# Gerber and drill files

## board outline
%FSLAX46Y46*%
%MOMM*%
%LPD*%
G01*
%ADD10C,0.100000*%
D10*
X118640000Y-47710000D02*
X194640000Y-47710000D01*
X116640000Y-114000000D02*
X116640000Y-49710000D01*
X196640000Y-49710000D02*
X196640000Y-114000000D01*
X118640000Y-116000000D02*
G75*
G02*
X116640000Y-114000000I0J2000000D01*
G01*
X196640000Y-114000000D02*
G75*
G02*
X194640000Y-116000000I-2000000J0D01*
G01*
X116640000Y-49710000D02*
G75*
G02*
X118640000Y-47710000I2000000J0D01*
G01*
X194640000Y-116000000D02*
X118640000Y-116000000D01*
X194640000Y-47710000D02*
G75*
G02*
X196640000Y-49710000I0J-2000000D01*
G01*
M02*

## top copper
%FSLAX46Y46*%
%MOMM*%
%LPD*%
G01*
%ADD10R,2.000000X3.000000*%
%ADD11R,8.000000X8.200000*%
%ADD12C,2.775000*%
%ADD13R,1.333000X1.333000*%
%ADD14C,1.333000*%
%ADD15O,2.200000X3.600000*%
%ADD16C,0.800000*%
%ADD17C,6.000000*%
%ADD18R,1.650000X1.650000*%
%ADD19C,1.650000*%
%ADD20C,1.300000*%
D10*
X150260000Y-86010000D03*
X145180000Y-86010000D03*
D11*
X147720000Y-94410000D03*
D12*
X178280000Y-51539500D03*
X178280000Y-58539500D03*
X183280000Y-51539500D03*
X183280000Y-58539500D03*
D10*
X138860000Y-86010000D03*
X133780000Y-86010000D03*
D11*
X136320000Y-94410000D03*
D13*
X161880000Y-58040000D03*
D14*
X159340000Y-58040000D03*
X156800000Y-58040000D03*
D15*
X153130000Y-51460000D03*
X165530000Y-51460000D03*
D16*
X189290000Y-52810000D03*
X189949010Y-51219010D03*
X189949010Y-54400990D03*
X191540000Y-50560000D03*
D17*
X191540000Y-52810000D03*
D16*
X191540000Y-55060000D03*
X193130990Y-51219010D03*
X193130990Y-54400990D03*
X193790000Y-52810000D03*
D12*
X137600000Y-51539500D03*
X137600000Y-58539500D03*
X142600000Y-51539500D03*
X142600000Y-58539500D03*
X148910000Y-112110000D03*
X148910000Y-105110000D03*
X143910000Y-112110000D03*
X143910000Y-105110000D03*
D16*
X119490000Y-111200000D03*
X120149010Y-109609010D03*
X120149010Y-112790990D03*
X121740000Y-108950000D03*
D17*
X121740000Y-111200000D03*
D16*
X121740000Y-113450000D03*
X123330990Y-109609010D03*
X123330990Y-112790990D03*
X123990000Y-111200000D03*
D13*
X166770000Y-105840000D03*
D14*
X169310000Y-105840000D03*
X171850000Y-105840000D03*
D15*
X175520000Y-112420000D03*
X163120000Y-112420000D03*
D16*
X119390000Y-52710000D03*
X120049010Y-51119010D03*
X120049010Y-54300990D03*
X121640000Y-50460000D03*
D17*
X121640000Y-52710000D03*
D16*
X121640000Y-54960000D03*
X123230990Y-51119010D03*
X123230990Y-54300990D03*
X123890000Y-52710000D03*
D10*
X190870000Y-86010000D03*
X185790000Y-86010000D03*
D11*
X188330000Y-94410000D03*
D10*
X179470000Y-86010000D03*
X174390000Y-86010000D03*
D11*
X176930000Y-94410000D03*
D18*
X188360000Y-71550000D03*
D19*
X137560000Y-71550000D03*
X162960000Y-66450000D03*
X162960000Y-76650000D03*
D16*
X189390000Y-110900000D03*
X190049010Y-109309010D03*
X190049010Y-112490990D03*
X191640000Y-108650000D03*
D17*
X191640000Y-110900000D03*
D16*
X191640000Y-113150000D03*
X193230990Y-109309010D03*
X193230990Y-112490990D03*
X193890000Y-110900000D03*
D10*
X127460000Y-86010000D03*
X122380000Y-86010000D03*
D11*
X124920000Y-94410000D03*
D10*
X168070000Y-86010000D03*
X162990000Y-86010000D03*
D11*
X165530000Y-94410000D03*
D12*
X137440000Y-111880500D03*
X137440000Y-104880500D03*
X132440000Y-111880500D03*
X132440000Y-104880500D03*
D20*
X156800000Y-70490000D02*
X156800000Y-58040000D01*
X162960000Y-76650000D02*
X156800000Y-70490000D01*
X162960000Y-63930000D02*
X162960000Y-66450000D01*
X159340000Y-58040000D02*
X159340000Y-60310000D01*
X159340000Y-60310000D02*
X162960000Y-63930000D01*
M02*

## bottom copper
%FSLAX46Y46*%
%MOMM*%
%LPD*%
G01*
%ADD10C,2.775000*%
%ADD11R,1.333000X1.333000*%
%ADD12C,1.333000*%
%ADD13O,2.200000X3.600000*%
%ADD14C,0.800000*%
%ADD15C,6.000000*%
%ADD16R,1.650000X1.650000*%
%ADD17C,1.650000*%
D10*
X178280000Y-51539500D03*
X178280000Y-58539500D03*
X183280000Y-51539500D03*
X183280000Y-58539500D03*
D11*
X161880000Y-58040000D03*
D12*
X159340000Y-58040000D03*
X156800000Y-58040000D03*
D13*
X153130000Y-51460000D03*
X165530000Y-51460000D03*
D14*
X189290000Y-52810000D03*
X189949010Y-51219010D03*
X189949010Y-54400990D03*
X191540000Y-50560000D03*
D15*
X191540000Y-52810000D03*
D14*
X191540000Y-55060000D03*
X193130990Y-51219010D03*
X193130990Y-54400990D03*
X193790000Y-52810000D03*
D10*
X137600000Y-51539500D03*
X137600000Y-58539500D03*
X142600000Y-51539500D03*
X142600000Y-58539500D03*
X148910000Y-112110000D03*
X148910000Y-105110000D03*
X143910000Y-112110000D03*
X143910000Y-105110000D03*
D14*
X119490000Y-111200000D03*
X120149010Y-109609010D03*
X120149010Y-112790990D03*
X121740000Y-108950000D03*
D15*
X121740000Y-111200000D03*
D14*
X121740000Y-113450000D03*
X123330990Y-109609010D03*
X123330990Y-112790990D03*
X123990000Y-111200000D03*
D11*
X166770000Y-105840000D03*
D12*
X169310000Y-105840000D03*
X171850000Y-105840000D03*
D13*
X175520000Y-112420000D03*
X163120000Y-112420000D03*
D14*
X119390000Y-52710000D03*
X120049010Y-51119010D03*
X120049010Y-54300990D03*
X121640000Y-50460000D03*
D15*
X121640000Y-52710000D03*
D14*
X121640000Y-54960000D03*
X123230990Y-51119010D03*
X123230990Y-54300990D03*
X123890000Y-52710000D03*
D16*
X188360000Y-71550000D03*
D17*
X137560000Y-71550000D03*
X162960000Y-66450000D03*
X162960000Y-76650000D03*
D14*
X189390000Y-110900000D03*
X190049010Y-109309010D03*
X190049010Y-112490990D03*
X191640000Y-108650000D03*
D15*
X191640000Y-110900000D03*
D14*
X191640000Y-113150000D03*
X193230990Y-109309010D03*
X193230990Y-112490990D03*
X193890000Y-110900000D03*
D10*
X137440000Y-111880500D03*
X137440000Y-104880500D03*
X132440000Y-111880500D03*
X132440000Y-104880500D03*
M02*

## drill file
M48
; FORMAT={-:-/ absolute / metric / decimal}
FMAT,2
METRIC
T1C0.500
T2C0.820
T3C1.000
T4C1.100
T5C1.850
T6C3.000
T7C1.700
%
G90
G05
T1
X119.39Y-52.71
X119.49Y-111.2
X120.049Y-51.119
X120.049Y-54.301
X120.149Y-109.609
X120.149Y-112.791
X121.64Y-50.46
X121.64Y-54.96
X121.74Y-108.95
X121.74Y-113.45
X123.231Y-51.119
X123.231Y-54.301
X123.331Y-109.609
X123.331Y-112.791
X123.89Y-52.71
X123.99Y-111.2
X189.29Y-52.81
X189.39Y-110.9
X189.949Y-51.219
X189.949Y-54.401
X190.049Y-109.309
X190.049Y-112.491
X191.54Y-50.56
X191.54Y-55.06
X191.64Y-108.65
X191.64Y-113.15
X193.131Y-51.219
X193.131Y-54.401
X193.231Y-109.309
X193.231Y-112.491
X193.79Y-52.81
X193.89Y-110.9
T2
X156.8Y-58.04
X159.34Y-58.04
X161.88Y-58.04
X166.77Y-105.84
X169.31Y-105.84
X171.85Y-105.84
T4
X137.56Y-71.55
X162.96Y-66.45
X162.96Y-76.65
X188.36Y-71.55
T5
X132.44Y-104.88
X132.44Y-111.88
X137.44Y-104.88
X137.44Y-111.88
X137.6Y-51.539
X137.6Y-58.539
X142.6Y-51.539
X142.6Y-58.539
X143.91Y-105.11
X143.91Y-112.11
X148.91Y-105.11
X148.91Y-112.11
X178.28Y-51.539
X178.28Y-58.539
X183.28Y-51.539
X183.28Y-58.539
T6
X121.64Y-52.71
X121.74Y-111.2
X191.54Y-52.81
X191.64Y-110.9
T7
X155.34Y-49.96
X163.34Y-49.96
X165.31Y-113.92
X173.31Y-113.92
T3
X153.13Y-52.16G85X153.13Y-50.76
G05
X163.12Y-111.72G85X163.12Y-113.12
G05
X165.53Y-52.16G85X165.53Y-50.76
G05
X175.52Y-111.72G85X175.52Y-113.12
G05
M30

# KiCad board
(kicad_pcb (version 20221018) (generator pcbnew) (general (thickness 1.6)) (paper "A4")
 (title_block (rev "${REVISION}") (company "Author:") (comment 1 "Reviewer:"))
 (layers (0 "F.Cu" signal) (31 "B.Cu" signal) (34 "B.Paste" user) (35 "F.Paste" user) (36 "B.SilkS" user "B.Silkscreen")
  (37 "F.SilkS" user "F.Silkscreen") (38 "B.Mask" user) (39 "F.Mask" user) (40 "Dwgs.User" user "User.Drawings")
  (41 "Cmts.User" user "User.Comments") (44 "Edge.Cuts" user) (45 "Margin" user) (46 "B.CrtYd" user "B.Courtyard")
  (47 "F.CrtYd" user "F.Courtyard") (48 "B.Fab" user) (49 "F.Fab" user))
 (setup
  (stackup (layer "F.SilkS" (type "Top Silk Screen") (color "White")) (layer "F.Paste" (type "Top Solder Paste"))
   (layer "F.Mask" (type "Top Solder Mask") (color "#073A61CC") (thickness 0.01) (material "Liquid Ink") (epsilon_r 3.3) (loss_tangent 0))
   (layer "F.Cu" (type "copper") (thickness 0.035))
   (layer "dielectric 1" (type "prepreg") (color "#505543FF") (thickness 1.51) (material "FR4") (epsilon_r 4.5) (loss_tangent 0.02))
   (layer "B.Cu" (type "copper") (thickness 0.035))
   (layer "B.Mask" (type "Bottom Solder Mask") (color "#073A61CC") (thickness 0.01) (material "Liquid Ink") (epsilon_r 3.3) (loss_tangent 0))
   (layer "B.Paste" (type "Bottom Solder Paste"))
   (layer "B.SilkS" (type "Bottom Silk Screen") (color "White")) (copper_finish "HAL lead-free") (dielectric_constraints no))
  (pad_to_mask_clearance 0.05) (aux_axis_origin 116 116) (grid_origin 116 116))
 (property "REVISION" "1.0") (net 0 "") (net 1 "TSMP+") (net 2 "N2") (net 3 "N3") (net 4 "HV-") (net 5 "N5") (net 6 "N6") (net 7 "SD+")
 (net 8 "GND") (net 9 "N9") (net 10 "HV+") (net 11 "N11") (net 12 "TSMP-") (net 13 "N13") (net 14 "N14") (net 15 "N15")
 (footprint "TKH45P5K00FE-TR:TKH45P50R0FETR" (layer "F.Cu") (at 147.72 90.21 180)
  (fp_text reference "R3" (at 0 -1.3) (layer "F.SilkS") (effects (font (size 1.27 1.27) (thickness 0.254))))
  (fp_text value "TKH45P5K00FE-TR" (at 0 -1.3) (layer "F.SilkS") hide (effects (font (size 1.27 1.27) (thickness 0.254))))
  (pad "1" smd rect (at -2.54 4.2 180) (size 2 3) (layers "F.Cu" "F.Paste" "F.Mask") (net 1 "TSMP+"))
  (pad "2" smd rect (at 2.54 4.2 180) (size 2 3) (layers "F.Cu" "F.Paste" "F.Mask") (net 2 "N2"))
  (pad "3" smd rect (at 0 -4.2 180) (size 8 8.2) (layers "F.Cu" "F.Paste" "F.Mask") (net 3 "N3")))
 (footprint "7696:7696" (layer "F.Cu") (at 178.28 58.5395)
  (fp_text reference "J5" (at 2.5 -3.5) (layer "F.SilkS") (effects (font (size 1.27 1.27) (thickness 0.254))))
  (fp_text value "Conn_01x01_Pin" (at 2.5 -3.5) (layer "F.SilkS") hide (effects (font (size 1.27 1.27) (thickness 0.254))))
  (pad "1" thru_hole circle (at 0 -7) (size 2.775 2.775) (drill 1.85) (layers "*.Cu" "*.Mask") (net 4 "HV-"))
  (pad "1" thru_hole circle (at 0 0) (size 2.775 2.775) (drill 1.85) (layers "*.Cu" "*.Mask") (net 4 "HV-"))
  (pad "1" thru_hole circle (at 5 -7) (size 2.775 2.775) (drill 1.85) (layers "*.Cu" "*.Mask") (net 4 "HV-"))
  (pad "1" thru_hole circle (at 5 0) (size 2.775 2.775) (drill 1.85) (layers "*.Cu" "*.Mask") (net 4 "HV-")))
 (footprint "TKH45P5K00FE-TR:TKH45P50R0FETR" (layer "F.Cu") (at 136.32 90.21 180)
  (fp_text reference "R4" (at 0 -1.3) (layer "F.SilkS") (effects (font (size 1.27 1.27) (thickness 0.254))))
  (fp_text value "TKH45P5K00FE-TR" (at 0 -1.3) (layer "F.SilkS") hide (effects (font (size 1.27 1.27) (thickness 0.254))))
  (pad "1" smd rect (at -2.54 4.2 180) (size 2 3) (layers "F.Cu" "F.Paste" "F.Mask") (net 2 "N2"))
  (pad "2" smd rect (at 2.54 4.2 180) (size 2 3) (layers "F.Cu" "F.Paste" "F.Mask") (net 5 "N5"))
  (pad "3" smd rect (at 0 -4.2 180) (size 8 8.2) (layers "F.Cu" "F.Paste" "F.Mask") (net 3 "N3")))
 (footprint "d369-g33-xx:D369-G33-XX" (layer "F.Cu") (at 161.88 58.04 90)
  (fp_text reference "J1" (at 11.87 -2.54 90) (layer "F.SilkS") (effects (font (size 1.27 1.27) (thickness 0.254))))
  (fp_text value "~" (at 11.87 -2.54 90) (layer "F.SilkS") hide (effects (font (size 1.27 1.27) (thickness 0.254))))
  (pad "" np_thru_hole circle (at 8.08 -6.54 90) (size 1.7 1.7) (drill 1.7) (layers "*.Cu" "*.Mask"))
  (pad "" np_thru_hole circle (at 8.08 1.46 90) (size 1.7 1.7) (drill 1.7) (layers "*.Cu" "*.Mask"))
  (pad "1" thru_hole rect (at 0 0 90) (size 1.333 1.333) (drill 0.82) (layers "*.Cu" "*.Mask") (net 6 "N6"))
  (pad "2" thru_hole circle (at 0 -2.54 90) (size 1.333 1.333) (drill 0.82) (layers "*.Cu" "*.Mask") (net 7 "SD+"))
  (pad "3" thru_hole circle (at 0 -5.08 90) (size 1.333 1.333) (drill 0.82) (layers "*.Cu" "*.Mask") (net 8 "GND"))
  (pad "MH" thru_hole oval (at 6.58 -8.75 90) (size 3.6 2.2) (drill oval 2.4 1) (layers "*.Cu" "*.Mask"))
  (pad "MH" thru_hole oval (at 6.58 3.65 90) (size 3.6 2.2) (drill oval 2.4 1) (layers "*.Cu" "*.Mask")))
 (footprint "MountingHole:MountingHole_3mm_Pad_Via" (layer "F.Cu") (at 191.54 52.81)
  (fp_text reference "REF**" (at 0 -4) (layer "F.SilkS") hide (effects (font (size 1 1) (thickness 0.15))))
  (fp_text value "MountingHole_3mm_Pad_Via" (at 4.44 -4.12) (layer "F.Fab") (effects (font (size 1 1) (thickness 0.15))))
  (pad "1" thru_hole circle (at -2.25 0) (size 0.8 0.8) (drill 0.5) (layers "*.Cu" "*.Mask") (zone_connect 2))
  (pad "1" thru_hole circle (at -1.59099 -1.59099) (size 0.8 0.8) (drill 0.5) (layers "*.Cu" "*.Mask") (zone_connect 2))
  (pad "1" thru_hole circle (at -1.59099 1.59099) (size 0.8 0.8) (drill 0.5) (layers "*.Cu" "*.Mask") (zone_connect 2))
  (pad "1" thru_hole circle (at 0 -2.25) (size 0.8 0.8) (drill 0.5) (layers "*.Cu" "*.Mask") (zone_connect 2))
  (pad "1" thru_hole circle (at 0 0) (size 6 6) (drill 3) (layers "*.Cu" "*.Mask"))
  (pad "1" thru_hole circle (at 0 2.25) (size 0.8 0.8) (drill 0.5) (layers "*.Cu" "*.Mask") (zone_connect 2))
  (pad "1" thru_hole circle (at 1.59099 -1.59099) (size 0.8 0.8) (drill 0.5) (layers "*.Cu" "*.Mask") (zone_connect 2))
  (pad "1" thru_hole circle (at 1.59099 1.59099) (size 0.8 0.8) (drill 0.5) (layers "*.Cu" "*.Mask") (zone_connect 2))
  (pad "1" thru_hole circle (at 2.25 0) (size 0.8 0.8) (drill 0.5) (layers "*.Cu" "*.Mask") (zone_connect 2)))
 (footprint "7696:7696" (layer "F.Cu") (at 137.6 58.5395)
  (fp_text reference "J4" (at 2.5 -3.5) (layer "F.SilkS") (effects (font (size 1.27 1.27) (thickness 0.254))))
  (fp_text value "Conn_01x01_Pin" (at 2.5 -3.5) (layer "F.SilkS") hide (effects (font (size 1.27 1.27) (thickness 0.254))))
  (pad "1" thru_hole circle (at 0 -7) (size 2.775 2.775) (drill 1.85) (layers "*.Cu" "*.Mask") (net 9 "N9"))
  (pad "1" thru_hole circle (at 0 0) (size 2.775 2.775) (drill 1.85) (layers "*.Cu" "*.Mask") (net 9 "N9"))
  (pad "1" thru_hole circle (at 5 -7) (size 2.775 2.775) (drill 1.85) (layers "*.Cu" "*.Mask") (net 9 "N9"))
  (pad "1" thru_hole circle (at 5 0) (size 2.775 2.775) (drill 1.85) (layers "*.Cu" "*.Mask") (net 9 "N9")))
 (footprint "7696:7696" (layer "F.Cu") (at 148.91 105.11 180)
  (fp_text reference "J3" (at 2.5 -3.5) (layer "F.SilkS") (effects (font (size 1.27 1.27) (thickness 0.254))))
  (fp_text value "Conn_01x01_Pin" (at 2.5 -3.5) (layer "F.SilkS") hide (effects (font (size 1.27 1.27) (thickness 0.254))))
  (pad "1" thru_hole circle (at 0 -7 180) (size 2.775 2.775) (drill 1.85) (layers "*.Cu" "*.Mask") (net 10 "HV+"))
  (pad "1" thru_hole circle (at 0 0 180) (size 2.775 2.775) (drill 1.85) (layers "*.Cu" "*.Mask") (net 10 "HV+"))
  (pad "1" thru_hole circle (at 5 -7 180) (size 2.775 2.775) (drill 1.85) (layers "*.Cu" "*.Mask") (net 10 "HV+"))
  (pad "1" thru_hole circle (at 5 0 180) (size 2.775 2.775) (drill 1.85) (layers "*.Cu" "*.Mask") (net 10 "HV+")))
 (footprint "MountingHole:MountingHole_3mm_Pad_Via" (layer "F.Cu") (at 121.74 111.2)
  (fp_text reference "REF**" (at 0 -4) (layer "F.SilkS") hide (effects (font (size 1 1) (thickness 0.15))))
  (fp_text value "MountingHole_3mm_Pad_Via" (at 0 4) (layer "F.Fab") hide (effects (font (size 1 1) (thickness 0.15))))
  (pad "1" thru_hole circle (at -2.25 0) (size 0.8 0.8) (drill 0.5) (layers "*.Cu" "*.Mask") (zone_connect 2))
  (pad "1" thru_hole circle (at -1.59099 -1.59099) (size 0.8 0.8) (drill 0.5) (layers "*.Cu" "*.Mask") (zone_connect 2))
  (pad "1" thru_hole circle (at -1.59099 1.59099) (size 0.8 0.8) (drill 0.5) (layers "*.Cu" "*.Mask") (zone_connect 2))
  (pad "1" thru_hole circle (at 0 -2.25) (size 0.8 0.8) (drill 0.5) (layers "*.Cu" "*.Mask") (zone_connect 2))
  (pad "1" thru_hole circle (at 0 0) (size 6 6) (drill 3) (layers "*.Cu" "*.Mask"))
  (pad "1" thru_hole circle (at 0 2.25) (size 0.8 0.8) (drill 0.5) (layers "*.Cu" "*.Mask") (zone_connect 2))
  (pad "1" thru_hole circle (at 1.59099 -1.59099) (size 0.8 0.8) (drill 0.5) (layers "*.Cu" "*.Mask") (zone_connect 2))
  (pad "1" thru_hole circle (at 1.59099 1.59099) (size 0.8 0.8) (drill 0.5) (layers "*.Cu" "*.Mask") (zone_connect 2))
  (pad "1" thru_hole circle (at 2.25 0) (size 0.8 0.8) (drill 0.5) (layers "*.Cu" "*.Mask") (zone_connect 2)))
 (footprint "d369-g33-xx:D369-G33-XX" (layer "F.Cu") (at 166.77 105.84 -90)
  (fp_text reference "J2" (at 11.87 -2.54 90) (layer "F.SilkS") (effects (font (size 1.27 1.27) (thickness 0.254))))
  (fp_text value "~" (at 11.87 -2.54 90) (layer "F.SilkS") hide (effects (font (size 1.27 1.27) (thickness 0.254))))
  (pad "" np_thru_hole circle (at 8.08 -6.54 270) (size 1.7 1.7) (drill 1.7) (layers "*.Cu" "*.Mask"))
  (pad "" np_thru_hole circle (at 8.08 1.46 270) (size 1.7 1.7) (drill 1.7) (layers "*.Cu" "*.Mask"))
  (pad "1" thru_hole rect (at 0 0 270) (size 1.333 1.333) (drill 0.82) (layers "*.Cu" "*.Mask") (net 1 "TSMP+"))
  (pad "2" thru_hole circle (at 0 -2.54 270) (size 1.333 1.333) (drill 0.82) (layers "*.Cu" "*.Mask") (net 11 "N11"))
  (pad "3" thru_hole circle (at 0 -5.08 270) (size 1.333 1.333) (drill 0.82) (layers "*.Cu" "*.Mask") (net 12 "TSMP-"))
  (pad "MH" thru_hole oval (at 6.58 -8.75 270) (size 3.6 2.2) (drill oval 2.4 1) (layers "*.Cu" "*.Mask"))
  (pad "MH" thru_hole oval (at 6.58 3.65 270) (size 3.6 2.2) (drill oval 2.4 1) (layers "*.Cu" "*.Mask")))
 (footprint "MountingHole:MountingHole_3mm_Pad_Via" (layer "F.Cu") (at 121.64 52.71)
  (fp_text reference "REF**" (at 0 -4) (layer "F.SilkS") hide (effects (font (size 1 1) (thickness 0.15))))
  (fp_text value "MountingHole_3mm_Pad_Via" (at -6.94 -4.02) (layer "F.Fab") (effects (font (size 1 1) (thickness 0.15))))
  (pad "1" thru_hole circle (at -2.25 0) (size 0.8 0.8) (drill 0.5) (layers "*.Cu" "*.Mask") (zone_connect 2))
  (pad "1" thru_hole circle (at -1.59099 -1.59099) (size 0.8 0.8) (drill 0.5) (layers "*.Cu" "*.Mask") (zone_connect 2))
  (pad "1" thru_hole circle (at -1.59099 1.59099) (size 0.8 0.8) (drill 0.5) (layers "*.Cu" "*.Mask") (zone_connect 2))
  (pad "1" thru_hole circle (at 0 -2.25) (size 0.8 0.8) (drill 0.5) (layers "*.Cu" "*.Mask") (zone_connect 2))
  (pad "1" thru_hole circle (at 0 0) (size 6 6) (drill 3) (layers "*.Cu" "*.Mask"))
  (pad "1" thru_hole circle (at 0 2.25) (size 0.8 0.8) (drill 0.5) (layers "*.Cu" "*.Mask") (zone_connect 2))
  (pad "1" thru_hole circle (at 1.59099 -1.59099) (size 0.8 0.8) (drill 0.5) (layers "*.Cu" "*.Mask") (zone_connect 2))
  (pad "1" thru_hole circle (at 1.59099 1.59099) (size 0.8 0.8) (drill 0.5) (layers "*.Cu" "*.Mask") (zone_connect 2))
  (pad "1" thru_hole circle (at 2.25 0) (size 0.8 0.8) (drill 0.5) (layers "*.Cu" "*.Mask") (zone_connect 2)))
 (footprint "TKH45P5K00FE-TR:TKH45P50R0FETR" (layer "F.Cu") (at 188.33 90.21 180)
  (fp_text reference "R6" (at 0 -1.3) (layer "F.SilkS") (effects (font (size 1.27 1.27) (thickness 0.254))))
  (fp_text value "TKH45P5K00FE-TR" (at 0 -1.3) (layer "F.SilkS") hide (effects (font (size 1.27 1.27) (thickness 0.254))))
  (pad "1" smd rect (at -2.54 4.2 180) (size 2 3) (layers "F.Cu" "F.Paste" "F.Mask") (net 12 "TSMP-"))
  (pad "2" smd rect (at 2.54 4.2 180) (size 2 3) (layers "F.Cu" "F.Paste" "F.Mask") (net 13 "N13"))
  (pad "3" smd rect (at 0 -4.2 180) (size 8 8.2) (layers "F.Cu" "F.Paste" "F.Mask") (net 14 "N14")))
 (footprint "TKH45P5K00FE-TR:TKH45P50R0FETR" (layer "F.Cu") (at 176.93 90.21 180)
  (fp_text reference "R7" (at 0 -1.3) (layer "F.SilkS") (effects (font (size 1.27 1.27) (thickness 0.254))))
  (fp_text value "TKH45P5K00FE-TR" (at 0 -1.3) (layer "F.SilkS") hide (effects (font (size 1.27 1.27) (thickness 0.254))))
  (pad "1" smd rect (at -2.54 4.2 180) (size 2 3) (layers "F.Cu" "F.Paste" "F.Mask") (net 13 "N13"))
  (pad "2" smd rect (at 2.54 4.2 180) (size 2 3) (layers "F.Cu" "F.Paste" "F.Mask") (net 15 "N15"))
  (pad "3" smd rect (at 0 -4.2 180) (size 8 8.2) (layers "F.Cu" "F.Paste" "F.Mask") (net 14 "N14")))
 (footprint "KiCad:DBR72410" (layer "F.Cu") (at 188.36 71.55 180)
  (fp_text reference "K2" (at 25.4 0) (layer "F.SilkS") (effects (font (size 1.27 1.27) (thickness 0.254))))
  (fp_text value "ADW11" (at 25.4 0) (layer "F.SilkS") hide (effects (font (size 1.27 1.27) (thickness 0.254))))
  (pad "1" thru_hole rect (at 0 0 180) (size 1.65 1.65) (drill 1.1) (layers "*.Cu" "*.Mask") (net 4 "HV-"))
  (pad "2" thru_hole circle (at 50.8 0 180) (size 1.65 1.65) (drill 1.1) (layers "*.Cu" "*.Mask") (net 9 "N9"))
  (pad "3" thru_hole circle (at 25.4 5.1 180) (size 1.65 1.65) (drill 1.1) (layers "*.Cu" "*.Mask") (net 7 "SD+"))
  (pad "4" thru_hole circle (at 25.4 -5.1 180) (size 1.65 1.65) (drill 1.1) (layers "*.Cu" "*.Mask") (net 8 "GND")))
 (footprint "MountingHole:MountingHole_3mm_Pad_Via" (layer "F.Cu") (at 191.64 110.9)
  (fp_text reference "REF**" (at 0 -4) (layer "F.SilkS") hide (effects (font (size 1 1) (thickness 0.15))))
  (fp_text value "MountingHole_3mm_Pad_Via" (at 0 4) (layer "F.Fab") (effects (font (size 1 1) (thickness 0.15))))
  (pad "1" thru_hole circle (at -2.25 0) (size 0.8 0.8) (drill 0.5) (layers "*.Cu" "*.Mask") (zone_connect 2))
  (pad "1" thru_hole circle (at -1.59099 -1.59099) (size 0.8 0.8) (drill 0.5) (layers "*.Cu" "*.Mask") (zone_connect 2))
  (pad "1" thru_hole circle (at -1.59099 1.59099) (size 0.8 0.8) (drill 0.5) (layers "*.Cu" "*.Mask") (zone_connect 2))
  (pad "1" thru_hole circle (at 0 -2.25) (size 0.8 0.8) (drill 0.5) (layers "*.Cu" "*.Mask") (zone_connect 2))
  (pad "1" thru_hole circle (at 0 0) (size 6 6) (drill 3) (layers "*.Cu" "*.Mask"))
  (pad "1" thru_hole circle (at 0 2.25) (size 0.8 0.8) (drill 0.5) (layers "*.Cu" "*.Mask") (zone_connect 2))
  (pad "1" thru_hole circle (at 1.59099 -1.59099) (size 0.8 0.8) (drill 0.5) (layers "*.Cu" "*.Mask") (zone_connect 2))
  (pad "1" thru_hole circle (at 1.59099 1.59099) (size 0.8 0.8) (drill 0.5) (layers "*.Cu" "*.Mask") (zone_connect 2))
  (pad "1" thru_hole circle (at 2.25 0) (size 0.8 0.8) (drill 0.5) (layers "*.Cu" "*.Mask") (zone_connect 2)))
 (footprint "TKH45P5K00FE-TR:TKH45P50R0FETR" (layer "F.Cu") (at 124.92 90.21 180)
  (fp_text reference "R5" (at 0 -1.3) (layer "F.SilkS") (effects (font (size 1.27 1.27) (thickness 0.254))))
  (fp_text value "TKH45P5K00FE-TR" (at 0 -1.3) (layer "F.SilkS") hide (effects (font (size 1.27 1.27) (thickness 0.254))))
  (pad "1" smd rect (at -2.54 4.2 180) (size 2 3) (layers "F.Cu" "F.Paste" "F.Mask") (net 5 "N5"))
  (pad "2" smd rect (at 2.54 4.2 180) (size 2 3) (layers "F.Cu" "F.Paste" "F.Mask") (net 10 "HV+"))
  (pad "3" smd rect (at 0 -4.2 180) (size 8 8.2) (layers "F.Cu" "F.Paste" "F.Mask") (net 3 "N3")))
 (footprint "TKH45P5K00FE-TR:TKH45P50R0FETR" (layer "F.Cu") (at 165.53 90.21 180)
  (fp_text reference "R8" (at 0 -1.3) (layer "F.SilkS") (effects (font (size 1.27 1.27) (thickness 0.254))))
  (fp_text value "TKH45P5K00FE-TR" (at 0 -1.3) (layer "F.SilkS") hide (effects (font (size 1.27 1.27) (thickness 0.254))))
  (pad "1" smd rect (at -2.54 4.2 180) (size 2 3) (layers "F.Cu" "F.Paste" "F.Mask") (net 15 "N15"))
  (pad "2" smd rect (at 2.54 4.2 180) (size 2 3) (layers "F.Cu" "F.Paste" "F.Mask") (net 4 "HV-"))
  (pad "3" smd rect (at 0 -4.2 180) (size 8 8.2) (layers "F.Cu" "F.Paste" "F.Mask") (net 14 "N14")))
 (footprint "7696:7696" (layer "F.Cu") (at 137.44 104.8805 180)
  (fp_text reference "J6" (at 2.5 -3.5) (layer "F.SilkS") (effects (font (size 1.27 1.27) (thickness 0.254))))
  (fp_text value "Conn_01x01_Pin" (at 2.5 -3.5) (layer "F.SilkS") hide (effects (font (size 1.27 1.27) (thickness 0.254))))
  (pad "1" thru_hole circle (at 0 -7 180) (size 2.775 2.775) (drill 1.85) (layers "*.Cu" "*.Mask") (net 10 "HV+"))
  (pad "1" thru_hole circle (at 0 0 180) (size 2.775 2.775) (drill 1.85) (layers "*.Cu" "*.Mask") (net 10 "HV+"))
  (pad "1" thru_hole circle (at 5 -7 180) (size 2.775 2.775) (drill 1.85) (layers "*.Cu" "*.Mask") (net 10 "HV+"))
  (pad "1" thru_hole circle (at 5 0 180) (size 2.775 2.775) (drill 1.85) (layers "*.Cu" "*.Mask") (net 10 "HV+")))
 (gr_line (start 118.64 47.71) (end 194.64 47.71) (stroke (width 0.1) (type default)) (layer "Edge.Cuts"))
 (gr_line (start 116.64 114) (end 116.64 49.71) (stroke (width 0.1) (type default)) (layer "Edge.Cuts"))
 (gr_line (start 196.64 49.71) (end 196.64 114) (stroke (width 0.1) (type default)) (layer "Edge.Cuts"))
 (gr_arc (start 118.64 116) (mid 117.225786 115.414214) (end 116.64 114) (stroke (width 0.1) (type default)) (layer "Edge.Cuts"))
 (gr_arc (start 196.64 114) (mid 196.054214 115.414214) (end 194.64 116) (stroke (width 0.1) (type default)) (layer "Edge.Cuts"))
 (gr_arc (start 116.64 49.71) (mid 117.225786 48.295786) (end 118.64 47.71) (stroke (width 0.1) (type default)) (layer "Edge.Cuts"))
 (gr_line (start 194.64 116) (end 118.64 116) (stroke (width 0.1) (type default)) (layer "Edge.Cuts"))
 (gr_arc (start 194.64 47.71) (mid 196.054214 48.295786) (end 196.64 49.71) (stroke (width 0.1) (type default)) (layer "Edge.Cuts"))
 (segment (start 156.8 70.49) (end 156.8 58.04) (width 1.3) (layer "F.Cu") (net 8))
 (segment (start 162.96 76.65) (end 156.8 70.49) (width 1.3) (layer "F.Cu") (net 8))
 (segment (start 162.96 63.93) (end 162.96 66.45) (width 1.3) (layer "F.Cu") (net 7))
 (segment (start 159.34 58.04) (end 159.34 60.31) (width 1.3) (layer "F.Cu") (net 7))
 (segment (start 159.34 60.31) (end 162.96 63.93) (width 1.3) (layer "F.Cu") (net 7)))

